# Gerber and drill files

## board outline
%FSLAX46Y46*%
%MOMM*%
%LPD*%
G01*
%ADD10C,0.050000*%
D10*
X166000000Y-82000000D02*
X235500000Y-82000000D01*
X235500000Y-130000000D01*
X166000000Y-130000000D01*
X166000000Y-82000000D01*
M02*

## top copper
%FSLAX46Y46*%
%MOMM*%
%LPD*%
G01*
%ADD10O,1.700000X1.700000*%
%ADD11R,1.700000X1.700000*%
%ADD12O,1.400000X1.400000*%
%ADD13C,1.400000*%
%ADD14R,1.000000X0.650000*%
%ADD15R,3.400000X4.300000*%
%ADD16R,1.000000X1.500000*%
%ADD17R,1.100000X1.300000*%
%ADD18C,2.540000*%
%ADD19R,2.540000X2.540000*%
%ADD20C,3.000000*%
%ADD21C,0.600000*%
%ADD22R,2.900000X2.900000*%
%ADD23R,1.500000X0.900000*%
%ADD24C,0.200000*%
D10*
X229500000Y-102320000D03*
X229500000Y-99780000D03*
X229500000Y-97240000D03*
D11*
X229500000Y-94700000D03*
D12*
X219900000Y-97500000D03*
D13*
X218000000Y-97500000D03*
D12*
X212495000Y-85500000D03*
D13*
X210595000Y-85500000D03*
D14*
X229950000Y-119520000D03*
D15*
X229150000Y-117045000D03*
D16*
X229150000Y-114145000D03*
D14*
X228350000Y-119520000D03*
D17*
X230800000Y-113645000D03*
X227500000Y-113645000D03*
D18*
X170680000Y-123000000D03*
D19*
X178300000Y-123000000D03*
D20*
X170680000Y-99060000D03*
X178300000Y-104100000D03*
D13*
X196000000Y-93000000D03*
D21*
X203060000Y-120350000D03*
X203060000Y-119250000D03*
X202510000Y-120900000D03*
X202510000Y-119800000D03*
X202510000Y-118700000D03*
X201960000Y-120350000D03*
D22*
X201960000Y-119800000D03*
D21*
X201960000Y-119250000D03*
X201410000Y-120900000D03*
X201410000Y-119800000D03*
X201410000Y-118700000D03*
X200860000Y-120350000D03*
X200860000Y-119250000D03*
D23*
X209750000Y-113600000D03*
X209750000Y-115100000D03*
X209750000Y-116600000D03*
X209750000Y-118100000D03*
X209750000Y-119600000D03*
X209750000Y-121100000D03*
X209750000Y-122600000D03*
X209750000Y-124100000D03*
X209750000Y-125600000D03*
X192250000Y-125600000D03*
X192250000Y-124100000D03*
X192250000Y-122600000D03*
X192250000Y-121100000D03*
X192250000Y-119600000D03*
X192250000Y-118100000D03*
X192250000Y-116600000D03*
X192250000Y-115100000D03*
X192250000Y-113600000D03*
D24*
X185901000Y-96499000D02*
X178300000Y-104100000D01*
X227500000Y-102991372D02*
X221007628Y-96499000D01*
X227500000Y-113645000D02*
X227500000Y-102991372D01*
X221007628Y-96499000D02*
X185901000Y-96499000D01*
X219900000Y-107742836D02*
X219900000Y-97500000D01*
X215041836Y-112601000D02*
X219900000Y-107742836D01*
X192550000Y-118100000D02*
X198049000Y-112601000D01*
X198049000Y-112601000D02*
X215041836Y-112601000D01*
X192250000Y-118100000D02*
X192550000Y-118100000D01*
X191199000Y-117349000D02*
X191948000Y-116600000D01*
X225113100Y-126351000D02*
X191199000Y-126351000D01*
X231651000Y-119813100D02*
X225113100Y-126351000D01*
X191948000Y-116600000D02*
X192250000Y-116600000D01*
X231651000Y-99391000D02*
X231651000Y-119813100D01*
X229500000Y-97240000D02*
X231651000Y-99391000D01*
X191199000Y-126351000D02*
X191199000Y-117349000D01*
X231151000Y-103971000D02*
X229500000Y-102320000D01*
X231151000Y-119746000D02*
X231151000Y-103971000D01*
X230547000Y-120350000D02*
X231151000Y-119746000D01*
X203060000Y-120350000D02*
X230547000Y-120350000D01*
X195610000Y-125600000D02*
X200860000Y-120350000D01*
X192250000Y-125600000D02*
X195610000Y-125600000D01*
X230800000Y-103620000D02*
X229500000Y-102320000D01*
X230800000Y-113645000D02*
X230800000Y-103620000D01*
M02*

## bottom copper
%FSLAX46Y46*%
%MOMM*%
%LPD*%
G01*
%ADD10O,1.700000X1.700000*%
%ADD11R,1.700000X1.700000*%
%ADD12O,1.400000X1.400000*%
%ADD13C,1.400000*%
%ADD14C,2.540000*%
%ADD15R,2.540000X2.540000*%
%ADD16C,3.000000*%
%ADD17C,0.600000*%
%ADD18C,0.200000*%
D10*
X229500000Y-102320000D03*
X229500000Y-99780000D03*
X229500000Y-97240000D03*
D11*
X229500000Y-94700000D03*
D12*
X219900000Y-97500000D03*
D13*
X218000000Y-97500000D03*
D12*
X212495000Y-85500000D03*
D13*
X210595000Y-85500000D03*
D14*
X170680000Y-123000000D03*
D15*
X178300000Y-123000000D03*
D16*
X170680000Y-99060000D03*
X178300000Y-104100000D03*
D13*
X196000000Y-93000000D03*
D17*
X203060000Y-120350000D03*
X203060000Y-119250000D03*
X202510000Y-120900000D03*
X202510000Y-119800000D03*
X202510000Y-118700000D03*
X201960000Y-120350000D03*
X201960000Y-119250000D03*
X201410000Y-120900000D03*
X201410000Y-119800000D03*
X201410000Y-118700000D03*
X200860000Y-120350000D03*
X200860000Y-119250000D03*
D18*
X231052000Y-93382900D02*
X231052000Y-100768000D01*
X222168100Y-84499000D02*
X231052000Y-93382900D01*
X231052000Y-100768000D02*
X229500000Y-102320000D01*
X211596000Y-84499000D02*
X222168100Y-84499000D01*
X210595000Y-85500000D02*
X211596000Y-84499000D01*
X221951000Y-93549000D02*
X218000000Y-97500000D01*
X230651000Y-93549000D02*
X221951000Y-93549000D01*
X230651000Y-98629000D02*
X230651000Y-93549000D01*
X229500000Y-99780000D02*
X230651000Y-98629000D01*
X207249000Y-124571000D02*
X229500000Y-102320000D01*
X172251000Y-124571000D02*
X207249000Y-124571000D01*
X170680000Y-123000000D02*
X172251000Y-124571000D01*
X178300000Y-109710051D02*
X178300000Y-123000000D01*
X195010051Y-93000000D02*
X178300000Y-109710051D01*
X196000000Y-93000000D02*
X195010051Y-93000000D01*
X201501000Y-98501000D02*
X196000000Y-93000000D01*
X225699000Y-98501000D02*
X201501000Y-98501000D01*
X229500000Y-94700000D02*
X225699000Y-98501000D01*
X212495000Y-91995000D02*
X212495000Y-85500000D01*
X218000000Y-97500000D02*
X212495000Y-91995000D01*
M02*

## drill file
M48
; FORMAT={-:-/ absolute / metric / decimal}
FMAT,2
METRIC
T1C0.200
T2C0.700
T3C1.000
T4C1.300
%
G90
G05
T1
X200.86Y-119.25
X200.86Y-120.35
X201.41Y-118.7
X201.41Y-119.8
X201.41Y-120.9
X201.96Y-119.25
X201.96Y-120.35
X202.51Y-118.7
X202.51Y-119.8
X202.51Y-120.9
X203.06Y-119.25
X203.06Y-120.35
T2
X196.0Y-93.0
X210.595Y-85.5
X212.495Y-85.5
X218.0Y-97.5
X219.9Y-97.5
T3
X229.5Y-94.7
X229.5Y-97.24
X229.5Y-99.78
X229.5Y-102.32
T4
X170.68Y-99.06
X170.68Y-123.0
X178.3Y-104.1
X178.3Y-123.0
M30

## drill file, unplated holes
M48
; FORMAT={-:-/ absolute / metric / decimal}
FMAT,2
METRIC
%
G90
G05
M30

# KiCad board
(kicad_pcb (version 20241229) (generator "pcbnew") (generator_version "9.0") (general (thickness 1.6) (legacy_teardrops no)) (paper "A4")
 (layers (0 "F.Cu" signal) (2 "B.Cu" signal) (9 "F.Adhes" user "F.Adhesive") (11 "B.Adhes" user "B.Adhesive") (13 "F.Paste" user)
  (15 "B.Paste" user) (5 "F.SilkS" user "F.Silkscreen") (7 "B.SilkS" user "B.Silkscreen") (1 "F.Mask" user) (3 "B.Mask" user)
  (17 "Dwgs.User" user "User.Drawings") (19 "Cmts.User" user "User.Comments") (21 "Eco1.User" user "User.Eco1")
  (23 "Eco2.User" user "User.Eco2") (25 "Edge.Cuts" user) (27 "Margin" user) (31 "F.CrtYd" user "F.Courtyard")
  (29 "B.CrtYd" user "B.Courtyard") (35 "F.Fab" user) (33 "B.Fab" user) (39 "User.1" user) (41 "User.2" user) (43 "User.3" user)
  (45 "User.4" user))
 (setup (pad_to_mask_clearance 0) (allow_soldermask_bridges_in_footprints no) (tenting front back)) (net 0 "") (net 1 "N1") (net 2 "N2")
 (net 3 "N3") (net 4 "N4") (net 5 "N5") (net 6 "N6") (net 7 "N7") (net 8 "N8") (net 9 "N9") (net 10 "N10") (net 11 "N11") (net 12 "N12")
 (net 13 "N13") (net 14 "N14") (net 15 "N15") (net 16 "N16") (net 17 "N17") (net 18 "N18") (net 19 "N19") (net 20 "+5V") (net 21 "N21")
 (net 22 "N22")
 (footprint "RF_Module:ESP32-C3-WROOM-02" (layer "F.Cu") (at 201 119.6)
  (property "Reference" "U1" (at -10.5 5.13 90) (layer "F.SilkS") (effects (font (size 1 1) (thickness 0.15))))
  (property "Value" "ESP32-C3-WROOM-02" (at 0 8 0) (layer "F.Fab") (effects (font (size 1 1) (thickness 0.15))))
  (pad "" smd rect (at -0.14 -0.9) (size 0.7 0.7) (layers "F.Paste"))
  (pad "" smd rect (at -0.14 0.2) (size 0.7 0.7) (layers "F.Paste"))
  (pad "" smd rect (at -0.14 1.3) (size 0.7 0.7) (layers "F.Paste"))
  (pad "" smd rect (at 0.96 -0.9) (size 0.7 0.7) (layers "F.Paste"))
  (pad "" smd rect (at 0.96 0.2) (size 0.7 0.7) (layers "F.Paste"))
  (pad "" smd rect (at 0.96 1.3) (size 0.7 0.7) (layers "F.Paste"))
  (pad "" smd rect (at 2.06 -0.9) (size 0.7 0.7) (layers "F.Paste"))
  (pad "" smd rect (at 2.06 0.2) (size 0.7 0.7) (layers "F.Paste"))
  (pad "" smd rect (at 2.06 1.3) (size 0.7 0.7) (layers "F.Paste"))
  (pad "1" smd rect (at -8.75 -6) (size 1.5 0.9) (layers "F.Cu" "F.Mask" "F.Paste") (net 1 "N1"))
  (pad "2" smd rect (at -8.75 -4.5) (size 1.5 0.9) (layers "F.Cu" "F.Mask" "F.Paste") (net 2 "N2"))
  (pad "3" smd rect (at -8.75 -3) (size 1.5 0.9) (layers "F.Cu" "F.Mask" "F.Paste") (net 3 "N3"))
  (pad "4" smd rect (at -8.75 -1.5) (size 1.5 0.9) (layers "F.Cu" "F.Mask" "F.Paste") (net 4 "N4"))
  (pad "5" smd rect (at -8.75 0) (size 1.5 0.9) (layers "F.Cu" "F.Mask" "F.Paste") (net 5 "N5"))
  (pad "6" smd rect (at -8.75 1.5) (size 1.5 0.9) (layers "F.Cu" "F.Mask" "F.Paste") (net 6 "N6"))
  (pad "7" smd rect (at -8.75 3) (size 1.5 0.9) (layers "F.Cu" "F.Mask" "F.Paste") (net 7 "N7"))
  (pad "8" smd rect (at -8.75 4.5) (size 1.5 0.9) (layers "F.Cu" "F.Mask" "F.Paste") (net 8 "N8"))
  (pad "9" smd rect (at -8.75 6) (size 1.5 0.9) (layers "F.Cu" "F.Mask" "F.Paste") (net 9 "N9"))
  (pad "10" smd rect (at 8.75 6) (size 1.5 0.9) (layers "F.Cu" "F.Mask" "F.Paste") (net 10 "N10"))
  (pad "11" smd rect (at 8.75 4.5) (size 1.5 0.9) (layers "F.Cu" "F.Mask" "F.Paste") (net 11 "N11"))
  (pad "12" smd rect (at 8.75 3) (size 1.5 0.9) (layers "F.Cu" "F.Mask" "F.Paste") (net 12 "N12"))
  (pad "13" smd rect (at 8.75 1.5) (size 1.5 0.9) (layers "F.Cu" "F.Mask" "F.Paste") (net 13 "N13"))
  (pad "14" smd rect (at 8.75 0) (size 1.5 0.9) (layers "F.Cu" "F.Mask" "F.Paste") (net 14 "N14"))
  (pad "15" smd rect (at 8.75 -1.5) (size 1.5 0.9) (layers "F.Cu" "F.Mask" "F.Paste") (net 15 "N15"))
  (pad "16" smd rect (at 8.75 -3) (size 1.5 0.9) (layers "F.Cu" "F.Mask" "F.Paste") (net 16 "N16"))
  (pad "17" smd rect (at 8.75 -4.5) (size 1.5 0.9) (layers "F.Cu" "F.Mask" "F.Paste") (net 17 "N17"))
  (pad "18" smd rect (at 8.75 -6) (size 1.5 0.9) (layers "F.Cu" "F.Mask" "F.Paste") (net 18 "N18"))
  (pad "19" thru_hole circle (at -0.14 -0.35) (size 0.6 0.6) (drill 0.2) (layers "*.Cu" "F.Mask") (remove_unused_layers no) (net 9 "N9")
   (zone_connect 2))
  (pad "19" thru_hole circle (at -0.14 0.75) (size 0.6 0.6) (drill 0.2) (layers "*.Cu" "F.Mask") (remove_unused_layers no) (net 9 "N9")
   (zone_connect 2))
  (pad "19" thru_hole circle (at 0.41 -0.9) (size 0.6 0.6) (drill 0.2) (layers "*.Cu" "F.Mask") (remove_unused_layers no) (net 9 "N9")
   (zone_connect 2))
  (pad "19" thru_hole circle (at 0.41 0.2) (size 0.6 0.6) (drill 0.2) (layers "*.Cu" "F.Mask") (remove_unused_layers no) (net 9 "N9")
   (zone_connect 2))
  (pad "19" thru_hole circle (at 0.41 1.3) (size 0.6 0.6) (drill 0.2) (layers "*.Cu" "F.Mask") (remove_unused_layers no) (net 9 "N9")
   (zone_connect 2))
  (pad "19" thru_hole circle (at 0.96 -0.35) (size 0.6 0.6) (drill 0.2) (layers "*.Cu" "F.Mask") (remove_unused_layers no) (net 9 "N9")
   (zone_connect 2))
  (pad "19" smd rect (at 0.96 0.2) (size 2.9 2.9) (layers "F.Cu" "F.Mask") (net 9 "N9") (zone_connect 2))
  (pad "19" thru_hole circle (at 0.96 0.75) (size 0.6 0.6) (drill 0.2) (layers "*.Cu" "F.Mask") (remove_unused_layers no) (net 9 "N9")
   (zone_connect 2))
  (pad "19" thru_hole circle (at 1.51 -0.9) (size 0.6 0.6) (drill 0.2) (layers "*.Cu" "F.Mask") (remove_unused_layers no) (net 9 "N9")
   (zone_connect 2))
  (pad "19" thru_hole circle (at 1.51 0.2) (size 0.6 0.6) (drill 0.2) (layers "*.Cu" "F.Mask") (remove_unused_layers no) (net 9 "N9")
   (zone_connect 2))
  (pad "19" thru_hole circle (at 1.51 1.3) (size 0.6 0.6) (drill 0.2) (layers "*.Cu" "F.Mask") (remove_unused_layers no) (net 9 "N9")
   (zone_connect 2))
  (pad "19" thru_hole circle (at 2.06 -0.35) (size 0.6 0.6) (drill 0.2) (layers "*.Cu" "F.Mask") (remove_unused_layers no) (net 9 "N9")
   (zone_connect 2))
  (pad "19" thru_hole circle (at 2.06 0.75) (size 0.6 0.6) (drill 0.2) (layers "*.Cu" "F.Mask") (remove_unused_layers no) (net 9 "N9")
   (zone_connect 2))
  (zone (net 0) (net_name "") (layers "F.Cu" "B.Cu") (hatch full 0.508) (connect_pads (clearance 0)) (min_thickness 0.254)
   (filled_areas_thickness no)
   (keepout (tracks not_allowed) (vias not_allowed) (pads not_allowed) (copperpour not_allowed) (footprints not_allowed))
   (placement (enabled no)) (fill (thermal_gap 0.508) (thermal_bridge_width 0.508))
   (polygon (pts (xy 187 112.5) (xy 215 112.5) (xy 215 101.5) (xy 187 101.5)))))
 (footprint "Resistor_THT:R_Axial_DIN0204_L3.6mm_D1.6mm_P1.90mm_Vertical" (layer "F.Cu") (at 210.595 85.5)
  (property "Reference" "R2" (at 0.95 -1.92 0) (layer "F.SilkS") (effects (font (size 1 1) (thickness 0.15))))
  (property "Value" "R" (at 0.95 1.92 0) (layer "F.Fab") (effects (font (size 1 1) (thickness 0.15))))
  (pad "1" thru_hole circle (at 0 0) (size 1.4 1.4) (drill 0.7) (layers "*.Cu" "*.Mask") (remove_unused_layers no) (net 9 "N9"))
  (pad "2" thru_hole oval (at 1.9 0) (size 1.4 1.4) (drill 0.7) (layers "*.Cu" "*.Mask") (remove_unused_layers no) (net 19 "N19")))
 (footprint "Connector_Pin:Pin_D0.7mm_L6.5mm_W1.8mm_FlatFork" (layer "F.Cu") (at 196 93)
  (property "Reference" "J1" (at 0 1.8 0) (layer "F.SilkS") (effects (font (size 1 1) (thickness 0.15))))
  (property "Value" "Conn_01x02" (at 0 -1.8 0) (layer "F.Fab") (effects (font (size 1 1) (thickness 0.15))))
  (pad "1" thru_hole circle (at 0 0) (size 1.4 1.4) (drill 0.7) (layers "*.Cu" "*.Mask") (remove_unused_layers no) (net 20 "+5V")))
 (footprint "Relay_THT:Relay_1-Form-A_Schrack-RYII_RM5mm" (layer "F.Cu") (at 178.3 123 90)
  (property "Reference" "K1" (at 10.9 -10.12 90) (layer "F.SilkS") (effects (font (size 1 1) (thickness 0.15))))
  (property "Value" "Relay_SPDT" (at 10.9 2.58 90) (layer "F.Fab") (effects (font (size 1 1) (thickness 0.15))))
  (pad "11" thru_hole circle (at 18.9 0 90) (size 3 3) (drill 1.3) (layers "*.Cu" "*.Mask") (remove_unused_layers no) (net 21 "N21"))
  (pad "14" thru_hole circle (at 23.94 -7.62 90) (size 3 3) (drill 1.3) (layers "*.Cu" "*.Mask") (remove_unused_layers no) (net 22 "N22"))
  (pad "A1" thru_hole rect (at 0 0 90) (size 2.54 2.54) (drill 1.3) (layers "*.Cu" "*.Mask") (remove_unused_layers no) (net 20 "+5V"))
  (pad "A2" thru_hole circle (at 0 -7.62 90) (size 2.54 2.54) (drill 1.3) (layers "*.Cu" "*.Mask") (remove_unused_layers no) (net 9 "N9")))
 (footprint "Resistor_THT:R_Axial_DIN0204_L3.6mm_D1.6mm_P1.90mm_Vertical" (layer "F.Cu") (at 218 97.5)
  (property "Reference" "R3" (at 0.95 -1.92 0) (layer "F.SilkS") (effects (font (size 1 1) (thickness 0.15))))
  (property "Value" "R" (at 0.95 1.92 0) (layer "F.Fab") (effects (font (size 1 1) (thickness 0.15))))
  (pad "1" thru_hole circle (at 0 0) (size 1.4 1.4) (drill 0.7) (layers "*.Cu" "*.Mask") (remove_unused_layers no) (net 19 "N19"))
  (pad "2" thru_hole oval (at 1.9 0) (size 1.4 1.4) (drill 0.7) (layers "*.Cu" "*.Mask") (remove_unused_layers no) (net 4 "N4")))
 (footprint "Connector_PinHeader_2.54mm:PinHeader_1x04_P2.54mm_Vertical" (layer "F.Cu") (at 229.5 94.7)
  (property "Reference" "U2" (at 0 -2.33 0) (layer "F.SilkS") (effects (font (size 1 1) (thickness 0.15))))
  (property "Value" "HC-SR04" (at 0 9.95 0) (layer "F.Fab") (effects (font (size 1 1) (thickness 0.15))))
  (pad "1" thru_hole rect (at 0 0) (size 1.7 1.7) (drill 1) (layers "*.Cu" "*.Mask") (remove_unused_layers no) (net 20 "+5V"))
  (pad "2" thru_hole oval (at 0 2.54) (size 1.7 1.7) (drill 1) (layers "*.Cu" "*.Mask") (remove_unused_layers no) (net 3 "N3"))
  (pad "3" thru_hole oval (at 0 5.08) (size 1.7 1.7) (drill 1) (layers "*.Cu" "*.Mask") (remove_unused_layers no) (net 19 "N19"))
  (pad "4" thru_hole oval (at 0 7.62) (size 1.7 1.7) (drill 1) (layers "*.Cu" "*.Mask") (remove_unused_layers no) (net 9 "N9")))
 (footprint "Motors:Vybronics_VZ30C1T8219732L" (layer "F.Cu") (at 229.15 117.995)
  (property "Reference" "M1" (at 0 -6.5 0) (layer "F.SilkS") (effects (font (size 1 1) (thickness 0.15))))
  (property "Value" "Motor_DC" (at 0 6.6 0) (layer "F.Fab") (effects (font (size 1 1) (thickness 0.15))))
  (pad "" smd rect (at -0.85 -2.315 270) (size 1.07 1.4) (layers "F.Paste"))
  (pad "" smd rect (at -0.85 -0.905 270) (size 1.07 1.4) (layers "F.Paste"))
  (pad "" smd rect (at -0.85 0.505 270) (size 1.07 1.4) (layers "F.Paste"))
  (pad "" smd rect (at 0.85 -2.315 270) (size 1.07 1.4) (layers "F.Paste"))
  (pad "" smd rect (at 0.85 -0.905 270) (size 1.07 1.4) (layers "F.Paste"))
  (pad "" smd rect (at 0.85 0.505 270) (size 1.07 1.4) (layers "F.Paste"))
  (pad "1" smd rect (at -1.65 -4.35 270) (size 1.3 1.1) (layers "F.Cu" "F.Mask" "F.Paste") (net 21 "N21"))
  (pad "2" smd rect (at 1.65 -4.35 270) (size 1.3 1.1) (layers "F.Cu" "F.Mask" "F.Paste") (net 9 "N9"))
  (pad "SH" smd rect (at -0.8 1.525) (size 1 0.65) (layers "F.Cu" "F.Mask" "F.Paste"))
  (pad "SH" smd rect (at 0 -3.85 270) (size 1.5 1) (layers "F.Cu" "F.Mask" "F.Paste"))
  (pad "SH" smd rect (at 0 -0.95 270) (size 4.3 3.4) (layers "F.Cu" "F.Mask"))
  (pad "SH" smd rect (at 0.8 1.525) (size 1 0.65) (layers "F.Cu" "F.Mask" "F.Paste")))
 (gr_rect (start 166 82) (end 235.5 130) (stroke (width 0.05) (type default)) (fill no) (layer "Edge.Cuts"))
 (segment (start 225.699 98.501) (end 201.501 98.501) (width 0.2) (layer "B.Cu") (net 20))
 (segment (start 195.010051 93) (end 178.3 109.710051) (width 0.2) (layer "B.Cu") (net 20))
 (segment (start 178.3 109.710051) (end 178.3 123) (width 0.2) (layer "B.Cu") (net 20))
 (segment (start 196 93) (end 195.010051 93) (width 0.2) (layer "B.Cu") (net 20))
 (segment (start 201.501 98.501) (end 196 93) (width 0.2) (layer "B.Cu") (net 20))
 (segment (start 229.5 94.7) (end 225.699 98.501) (width 0.2) (layer "B.Cu") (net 20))
 (segment (start 227.5 113.645) (end 227.5 102.991372) (width 0.2) (layer "F.Cu") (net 21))
 (segment (start 227.5 102.991372) (end 221.007628 96.499) (width 0.2) (layer "F.Cu") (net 21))
 (segment (start 221.007628 96.499) (end 185.901 96.499) (width 0.2) (layer "F.Cu") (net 21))
 (segment (start 185.901 96.499) (end 178.3 104.1) (width 0.2) (layer "F.Cu") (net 21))
 (segment (start 203.06 120.35) (end 230.547 120.35) (width 0.2) (layer "F.Cu") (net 9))
 (segment (start 230.547 120.35) (end 231.151 119.746) (width 0.2) (layer "F.Cu") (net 9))
 (segment (start 231.151 119.746) (end 231.151 103.971) (width 0.2) (layer "F.Cu") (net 9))
 (segment (start 231.151 103.971) (end 229.5 102.32) (width 0.2) (layer "F.Cu") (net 9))
 (segment (start 192.25 125.6) (end 195.61 125.6) (width 0.2) (layer "F.Cu") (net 9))
 (segment (start 195.61 125.6) (end 200.86 120.35) (width 0.2) (layer "F.Cu") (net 9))
 (segment (start 230.8 103.62) (end 229.5 102.32) (width 0.2) (layer "F.Cu") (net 9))
 (segment (start 230.8 113.645) (end 230.8 103.62) (width 0.2) (layer "F.Cu") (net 9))
 (segment (start 231.052 100.768) (end 229.5 102.32) (width 0.2) (layer "B.Cu") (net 9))
 (segment (start 170.68 123) (end 172.251 124.571) (width 0.2) (layer "B.Cu") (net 9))
 (segment (start 207.249 124.571) (end 229.5 102.32) (width 0.2) (layer "B.Cu") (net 9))
 (segment (start 172.251 124.571) (end 207.249 124.571) (width 0.2) (layer "B.Cu") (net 9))
 (segment (start 210.595 85.5) (end 211.596 84.499) (width 0.2) (layer "B.Cu") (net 9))
 (segment (start 211.596 84.499) (end 222.1681 84.499) (width 0.2) (layer "B.Cu") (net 9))
 (segment (start 222.1681 84.499) (end 231.052 93.3829) (width 0.2) (layer "B.Cu") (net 9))
 (segment (start 231.052 93.3829) (end 231.052 100.768) (width 0.2) (layer "B.Cu") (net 9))
 (segment (start 229.5 99.78) (end 230.651 98.629) (width 0.2) (layer "B.Cu") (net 19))
 (segment (start 221.951 93.549) (end 218 97.5) (width 0.2) (layer "B.Cu") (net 19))
 (segment (start 230.651 98.629) (end 230.651 93.549) (width 0.2) (layer "B.Cu") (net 19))
 (segment (start 218 97.5) (end 212.495 91.995) (width 0.2) (layer "B.Cu") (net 19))
 (segment (start 212.495 91.995) (end 212.495 85.5) (width 0.2) (layer "B.Cu") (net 19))
 (segment (start 230.651 93.549) (end 221.951 93.549) (width 0.2) (layer "B.Cu") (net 19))
 (segment (start 219.9 107.742836) (end 219.9 97.5) (width 0.2) (layer "F.Cu") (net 4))
 (segment (start 192.55 118.1) (end 198.049 112.601) (width 0.2) (layer "F.Cu") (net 4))
 (segment (start 192.25 118.1) (end 192.55 118.1) (width 0.2) (layer "F.Cu") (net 4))
 (segment (start 215.041836 112.601) (end 219.9 107.742836) (width 0.2) (layer "F.Cu") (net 4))
 (segment (start 198.049 112.601) (end 215.041836 112.601) (width 0.2) (layer "F.Cu") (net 4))
 (segment (start 191.199 126.351) (end 191.199 117.349) (width 0.2) (layer "F.Cu") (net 3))
 (segment (start 229.5 97.24) (end 231.651 99.391) (width 0.2) (layer "F.Cu") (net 3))
 (segment (start 231.651 99.391) (end 231.651 119.8131) (width 0.2) (layer "F.Cu") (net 3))
 (segment (start 231.651 119.8131) (end 225.1131 126.351) (width 0.2) (layer "F.Cu") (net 3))
 (segment (start 191.948 116.6) (end 192.25 116.6) (width 0.2) (layer "F.Cu") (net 3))
 (segment (start 191.199 117.349) (end 191.948 116.6) (width 0.2) (layer "F.Cu") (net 3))
 (segment (start 225.1131 126.351) (end 191.199 126.351) (width 0.2) (layer "F.Cu") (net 3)))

